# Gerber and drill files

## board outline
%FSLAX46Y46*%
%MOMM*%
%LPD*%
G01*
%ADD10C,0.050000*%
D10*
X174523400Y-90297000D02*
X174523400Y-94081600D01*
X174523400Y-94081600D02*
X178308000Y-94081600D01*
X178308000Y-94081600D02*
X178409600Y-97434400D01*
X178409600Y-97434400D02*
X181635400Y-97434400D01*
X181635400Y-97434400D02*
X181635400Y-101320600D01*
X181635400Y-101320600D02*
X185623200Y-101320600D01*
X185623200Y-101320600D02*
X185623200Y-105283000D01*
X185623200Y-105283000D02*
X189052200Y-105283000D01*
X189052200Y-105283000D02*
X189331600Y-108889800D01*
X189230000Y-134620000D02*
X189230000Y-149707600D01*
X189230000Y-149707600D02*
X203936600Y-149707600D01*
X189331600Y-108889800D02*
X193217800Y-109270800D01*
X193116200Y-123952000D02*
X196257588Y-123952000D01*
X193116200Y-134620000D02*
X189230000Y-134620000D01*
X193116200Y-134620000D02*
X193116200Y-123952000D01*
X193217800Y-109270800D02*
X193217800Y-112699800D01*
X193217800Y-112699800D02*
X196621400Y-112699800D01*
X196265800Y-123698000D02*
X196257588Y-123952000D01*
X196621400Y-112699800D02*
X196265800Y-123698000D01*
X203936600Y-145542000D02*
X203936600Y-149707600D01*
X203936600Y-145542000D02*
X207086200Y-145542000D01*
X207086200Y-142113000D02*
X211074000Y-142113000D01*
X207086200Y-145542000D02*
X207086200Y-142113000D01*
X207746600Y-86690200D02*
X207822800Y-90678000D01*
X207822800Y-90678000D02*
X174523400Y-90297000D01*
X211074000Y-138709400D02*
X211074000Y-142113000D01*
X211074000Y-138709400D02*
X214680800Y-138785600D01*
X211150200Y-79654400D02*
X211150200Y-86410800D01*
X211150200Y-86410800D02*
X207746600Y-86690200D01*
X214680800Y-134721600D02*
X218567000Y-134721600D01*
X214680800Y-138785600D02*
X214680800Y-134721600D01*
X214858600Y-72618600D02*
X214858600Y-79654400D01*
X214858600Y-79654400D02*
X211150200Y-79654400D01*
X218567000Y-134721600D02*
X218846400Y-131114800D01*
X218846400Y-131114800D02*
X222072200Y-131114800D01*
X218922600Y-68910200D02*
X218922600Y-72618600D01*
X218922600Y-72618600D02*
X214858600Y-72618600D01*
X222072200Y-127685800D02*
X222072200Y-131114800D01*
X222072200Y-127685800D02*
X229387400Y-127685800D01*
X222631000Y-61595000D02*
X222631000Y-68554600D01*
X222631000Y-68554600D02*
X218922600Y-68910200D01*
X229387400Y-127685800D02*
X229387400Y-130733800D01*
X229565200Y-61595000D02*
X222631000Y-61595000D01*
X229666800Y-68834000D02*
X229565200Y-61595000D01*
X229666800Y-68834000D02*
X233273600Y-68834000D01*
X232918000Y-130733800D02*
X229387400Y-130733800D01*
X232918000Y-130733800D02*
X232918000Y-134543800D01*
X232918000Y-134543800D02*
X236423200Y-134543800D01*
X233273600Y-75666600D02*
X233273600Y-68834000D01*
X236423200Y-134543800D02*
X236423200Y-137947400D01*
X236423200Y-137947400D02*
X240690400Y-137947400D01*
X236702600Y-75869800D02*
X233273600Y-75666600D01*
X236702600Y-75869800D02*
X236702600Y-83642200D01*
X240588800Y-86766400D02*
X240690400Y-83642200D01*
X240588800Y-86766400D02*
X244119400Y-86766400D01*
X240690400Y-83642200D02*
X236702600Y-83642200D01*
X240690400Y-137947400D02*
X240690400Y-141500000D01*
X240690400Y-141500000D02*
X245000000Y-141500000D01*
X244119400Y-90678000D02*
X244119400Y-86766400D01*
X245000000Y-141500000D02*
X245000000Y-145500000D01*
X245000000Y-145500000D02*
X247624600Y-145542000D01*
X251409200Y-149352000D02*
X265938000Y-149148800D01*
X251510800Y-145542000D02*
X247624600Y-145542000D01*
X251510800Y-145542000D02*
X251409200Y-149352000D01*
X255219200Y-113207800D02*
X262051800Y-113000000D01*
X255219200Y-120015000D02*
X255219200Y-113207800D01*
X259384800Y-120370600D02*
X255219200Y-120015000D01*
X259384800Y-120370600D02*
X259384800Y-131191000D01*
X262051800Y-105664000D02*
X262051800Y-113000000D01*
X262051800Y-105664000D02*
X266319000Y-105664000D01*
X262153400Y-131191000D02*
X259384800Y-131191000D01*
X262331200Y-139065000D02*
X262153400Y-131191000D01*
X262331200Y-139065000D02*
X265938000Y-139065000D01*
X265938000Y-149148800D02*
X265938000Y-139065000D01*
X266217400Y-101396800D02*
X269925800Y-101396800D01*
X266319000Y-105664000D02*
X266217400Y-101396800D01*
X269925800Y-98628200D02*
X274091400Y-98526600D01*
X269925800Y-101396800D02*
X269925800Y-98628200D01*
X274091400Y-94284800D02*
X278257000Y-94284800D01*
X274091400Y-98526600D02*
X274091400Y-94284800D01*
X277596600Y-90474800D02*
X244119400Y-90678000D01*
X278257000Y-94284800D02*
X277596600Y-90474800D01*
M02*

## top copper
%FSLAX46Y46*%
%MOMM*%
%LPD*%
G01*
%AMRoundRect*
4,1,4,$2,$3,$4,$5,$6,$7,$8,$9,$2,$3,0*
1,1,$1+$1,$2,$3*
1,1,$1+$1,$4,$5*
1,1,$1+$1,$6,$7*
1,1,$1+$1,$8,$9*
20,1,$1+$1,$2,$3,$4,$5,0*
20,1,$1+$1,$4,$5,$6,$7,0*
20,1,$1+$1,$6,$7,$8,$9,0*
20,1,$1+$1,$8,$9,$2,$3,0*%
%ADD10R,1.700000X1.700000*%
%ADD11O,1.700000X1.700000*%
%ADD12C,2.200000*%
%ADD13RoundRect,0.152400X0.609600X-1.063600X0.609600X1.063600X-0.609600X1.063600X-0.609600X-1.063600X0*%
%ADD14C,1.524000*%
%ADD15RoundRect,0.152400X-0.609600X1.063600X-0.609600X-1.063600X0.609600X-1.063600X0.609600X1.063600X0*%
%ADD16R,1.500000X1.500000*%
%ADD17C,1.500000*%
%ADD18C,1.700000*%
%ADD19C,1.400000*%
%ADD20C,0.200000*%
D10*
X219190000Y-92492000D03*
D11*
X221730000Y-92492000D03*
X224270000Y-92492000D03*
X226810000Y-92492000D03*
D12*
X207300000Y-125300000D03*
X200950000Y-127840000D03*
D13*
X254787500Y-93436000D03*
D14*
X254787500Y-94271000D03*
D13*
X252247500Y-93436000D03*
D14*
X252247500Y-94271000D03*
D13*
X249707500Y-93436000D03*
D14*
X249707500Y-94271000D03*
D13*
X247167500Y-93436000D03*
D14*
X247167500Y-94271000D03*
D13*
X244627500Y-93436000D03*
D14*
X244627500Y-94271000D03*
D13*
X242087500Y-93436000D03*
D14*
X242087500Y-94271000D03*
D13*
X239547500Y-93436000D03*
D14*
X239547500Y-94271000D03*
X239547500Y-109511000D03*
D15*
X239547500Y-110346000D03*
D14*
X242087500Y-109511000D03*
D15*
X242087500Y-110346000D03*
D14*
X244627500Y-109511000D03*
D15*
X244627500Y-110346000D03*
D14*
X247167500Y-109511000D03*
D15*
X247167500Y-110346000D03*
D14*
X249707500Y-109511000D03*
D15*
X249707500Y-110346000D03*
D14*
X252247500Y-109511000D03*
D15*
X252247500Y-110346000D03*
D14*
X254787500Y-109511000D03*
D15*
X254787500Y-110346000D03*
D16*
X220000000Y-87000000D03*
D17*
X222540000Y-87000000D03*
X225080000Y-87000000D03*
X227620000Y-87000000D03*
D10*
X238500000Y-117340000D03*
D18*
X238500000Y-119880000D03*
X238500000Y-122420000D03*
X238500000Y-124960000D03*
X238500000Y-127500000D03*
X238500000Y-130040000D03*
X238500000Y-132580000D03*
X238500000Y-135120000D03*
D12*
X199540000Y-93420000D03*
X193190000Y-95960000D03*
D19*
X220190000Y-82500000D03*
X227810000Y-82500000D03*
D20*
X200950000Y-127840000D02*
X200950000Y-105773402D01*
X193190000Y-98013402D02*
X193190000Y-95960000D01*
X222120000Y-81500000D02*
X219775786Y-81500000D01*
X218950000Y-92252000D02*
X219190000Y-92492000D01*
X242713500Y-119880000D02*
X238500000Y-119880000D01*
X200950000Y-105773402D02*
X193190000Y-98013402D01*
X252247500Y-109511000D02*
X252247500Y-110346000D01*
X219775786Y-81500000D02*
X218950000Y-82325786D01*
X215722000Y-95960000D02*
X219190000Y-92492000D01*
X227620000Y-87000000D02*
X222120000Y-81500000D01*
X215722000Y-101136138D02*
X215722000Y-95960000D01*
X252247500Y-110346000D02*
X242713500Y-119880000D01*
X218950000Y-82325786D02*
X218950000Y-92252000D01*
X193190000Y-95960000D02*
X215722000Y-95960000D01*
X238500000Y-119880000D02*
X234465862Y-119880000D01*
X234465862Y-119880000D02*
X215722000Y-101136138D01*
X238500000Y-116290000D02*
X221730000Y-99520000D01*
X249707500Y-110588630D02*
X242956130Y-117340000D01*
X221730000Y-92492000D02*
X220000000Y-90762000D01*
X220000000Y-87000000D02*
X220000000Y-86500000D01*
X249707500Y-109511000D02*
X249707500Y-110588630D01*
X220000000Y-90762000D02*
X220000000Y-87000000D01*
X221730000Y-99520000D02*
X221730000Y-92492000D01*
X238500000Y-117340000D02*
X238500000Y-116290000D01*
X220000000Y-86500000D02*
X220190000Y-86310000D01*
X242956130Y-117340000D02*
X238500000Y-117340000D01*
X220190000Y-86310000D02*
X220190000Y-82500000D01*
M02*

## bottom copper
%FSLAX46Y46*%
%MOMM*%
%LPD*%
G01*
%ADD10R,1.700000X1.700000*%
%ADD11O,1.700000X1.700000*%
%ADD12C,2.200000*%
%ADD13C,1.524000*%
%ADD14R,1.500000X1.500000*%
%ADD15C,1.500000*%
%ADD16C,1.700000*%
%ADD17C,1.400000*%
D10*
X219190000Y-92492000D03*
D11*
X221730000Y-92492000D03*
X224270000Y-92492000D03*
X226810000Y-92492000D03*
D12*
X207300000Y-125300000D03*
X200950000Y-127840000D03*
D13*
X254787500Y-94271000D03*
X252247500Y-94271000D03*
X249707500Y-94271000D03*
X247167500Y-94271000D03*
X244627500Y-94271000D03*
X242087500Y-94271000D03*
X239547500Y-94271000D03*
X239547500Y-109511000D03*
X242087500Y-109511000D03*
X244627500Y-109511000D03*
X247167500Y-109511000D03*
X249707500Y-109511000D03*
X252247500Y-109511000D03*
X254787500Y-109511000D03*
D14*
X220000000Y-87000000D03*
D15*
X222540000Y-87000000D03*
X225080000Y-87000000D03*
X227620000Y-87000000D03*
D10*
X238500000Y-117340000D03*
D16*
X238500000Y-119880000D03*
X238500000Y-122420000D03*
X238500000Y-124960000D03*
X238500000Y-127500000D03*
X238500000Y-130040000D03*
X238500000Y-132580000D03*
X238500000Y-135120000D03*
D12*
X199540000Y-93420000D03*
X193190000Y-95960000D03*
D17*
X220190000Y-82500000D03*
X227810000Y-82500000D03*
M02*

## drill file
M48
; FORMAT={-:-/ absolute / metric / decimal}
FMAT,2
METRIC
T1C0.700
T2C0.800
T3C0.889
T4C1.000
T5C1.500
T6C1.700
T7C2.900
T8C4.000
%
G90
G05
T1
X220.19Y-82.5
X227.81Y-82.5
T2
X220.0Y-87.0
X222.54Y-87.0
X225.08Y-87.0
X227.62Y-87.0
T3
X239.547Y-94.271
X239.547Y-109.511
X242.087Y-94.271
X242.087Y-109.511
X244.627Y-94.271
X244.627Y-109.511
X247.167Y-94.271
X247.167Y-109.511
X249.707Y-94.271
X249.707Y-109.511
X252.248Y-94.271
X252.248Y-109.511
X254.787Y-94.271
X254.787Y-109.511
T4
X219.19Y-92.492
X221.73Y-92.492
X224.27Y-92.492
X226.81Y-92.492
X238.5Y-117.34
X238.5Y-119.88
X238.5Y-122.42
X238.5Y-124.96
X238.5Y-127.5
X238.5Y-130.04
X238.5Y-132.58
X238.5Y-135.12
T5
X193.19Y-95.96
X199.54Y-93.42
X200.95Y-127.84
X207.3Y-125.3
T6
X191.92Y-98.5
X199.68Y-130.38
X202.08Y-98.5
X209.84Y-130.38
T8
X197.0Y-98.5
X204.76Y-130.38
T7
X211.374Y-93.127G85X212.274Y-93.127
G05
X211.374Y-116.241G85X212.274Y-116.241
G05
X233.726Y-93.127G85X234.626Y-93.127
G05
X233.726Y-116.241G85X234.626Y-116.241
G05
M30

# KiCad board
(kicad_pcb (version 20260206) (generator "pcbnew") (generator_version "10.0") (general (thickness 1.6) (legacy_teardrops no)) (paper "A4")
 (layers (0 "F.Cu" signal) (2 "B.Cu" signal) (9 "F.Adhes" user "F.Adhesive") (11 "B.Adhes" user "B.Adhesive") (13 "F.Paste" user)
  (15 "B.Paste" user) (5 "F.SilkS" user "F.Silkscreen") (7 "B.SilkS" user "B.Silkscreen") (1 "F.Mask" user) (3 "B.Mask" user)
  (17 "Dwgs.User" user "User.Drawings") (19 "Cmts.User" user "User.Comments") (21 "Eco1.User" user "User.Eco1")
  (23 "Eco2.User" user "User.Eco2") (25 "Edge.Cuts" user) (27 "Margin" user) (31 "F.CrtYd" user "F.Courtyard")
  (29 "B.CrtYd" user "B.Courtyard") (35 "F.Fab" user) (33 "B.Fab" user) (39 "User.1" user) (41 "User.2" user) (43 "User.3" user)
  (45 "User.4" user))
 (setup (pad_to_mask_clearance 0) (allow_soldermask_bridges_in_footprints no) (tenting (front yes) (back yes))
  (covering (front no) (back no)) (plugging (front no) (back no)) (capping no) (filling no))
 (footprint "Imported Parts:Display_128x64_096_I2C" (layer "F.Cu") (at 223 92.492)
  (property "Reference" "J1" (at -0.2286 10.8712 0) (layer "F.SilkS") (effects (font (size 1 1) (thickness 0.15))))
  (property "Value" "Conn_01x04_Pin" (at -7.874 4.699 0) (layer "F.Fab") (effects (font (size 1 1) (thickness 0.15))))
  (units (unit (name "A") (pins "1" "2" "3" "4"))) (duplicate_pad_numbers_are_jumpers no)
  (pad "" np_thru_hole oval (at -11.176 0.635) (size 3.8 2.9) (drill oval 3.8 2.9) (layers "*.Cu" "*.Mask"))
  (pad "" np_thru_hole oval (at -11.176 23.749) (size 3.8 2.9) (drill oval 3.8 2.9) (layers "*.Cu" "*.Mask"))
  (pad "" np_thru_hole oval (at 11.176 0.635) (size 3.8 2.9) (drill oval 3.8 2.9) (layers "*.Cu" "*.Mask"))
  (pad "" np_thru_hole oval (at 11.176 23.749) (size 3.8 2.9) (drill oval 3.8 2.9) (layers "*.Cu" "*.Mask"))
  (pad "1" thru_hole rect (at -3.81 0 90) (size 1.7 1.7) (drill 1) (layers "*.Cu" "*.Mask") (remove_unused_layers no) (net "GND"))
  (pad "2" thru_hole oval (at -1.27 0 90) (size 1.7 1.7) (drill 1) (layers "*.Cu" "*.Mask") (remove_unused_layers no) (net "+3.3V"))
  (pad "3" thru_hole oval (at 1.27 0 90) (size 1.7 1.7) (drill 1) (layers "*.Cu" "*.Mask") (remove_unused_layers no)
   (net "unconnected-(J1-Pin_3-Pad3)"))
  (pad "4" thru_hole oval (at 3.81 0 90) (size 1.7 1.7) (drill 1) (layers "*.Cu" "*.Mask") (remove_unused_layers no)
   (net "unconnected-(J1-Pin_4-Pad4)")))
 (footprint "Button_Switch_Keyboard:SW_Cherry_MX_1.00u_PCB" (layer "F.Cu") (at 207.3 125.3)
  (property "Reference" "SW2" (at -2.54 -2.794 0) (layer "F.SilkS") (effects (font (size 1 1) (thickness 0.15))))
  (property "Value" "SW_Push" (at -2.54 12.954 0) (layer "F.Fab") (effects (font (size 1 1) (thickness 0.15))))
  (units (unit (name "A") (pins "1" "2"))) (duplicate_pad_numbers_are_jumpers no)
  (pad "" np_thru_hole circle (at -7.62 5.08) (size 1.7 1.7) (drill 1.7) (layers "*.Cu" "*.Mask"))
  (pad "" np_thru_hole circle (at -2.54 5.08) (size 4 4) (drill 4) (layers "*.Cu" "*.Mask"))
  (pad "" np_thru_hole circle (at 2.54 5.08) (size 1.7 1.7) (drill 1.7) (layers "*.Cu" "*.Mask"))
  (pad "1" thru_hole circle (at 0 0) (size 2.2 2.2) (drill 1.5) (layers "*.Cu" "*.Mask") (remove_unused_layers no)
   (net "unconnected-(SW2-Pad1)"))
  (pad "2" thru_hole circle (at -6.35 2.54) (size 2.2 2.2) (drill 1.5) (layers "*.Cu" "*.Mask") (remove_unused_layers no) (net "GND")))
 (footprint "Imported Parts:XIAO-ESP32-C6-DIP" (layer "F.Cu") (at 247.1675 101.891)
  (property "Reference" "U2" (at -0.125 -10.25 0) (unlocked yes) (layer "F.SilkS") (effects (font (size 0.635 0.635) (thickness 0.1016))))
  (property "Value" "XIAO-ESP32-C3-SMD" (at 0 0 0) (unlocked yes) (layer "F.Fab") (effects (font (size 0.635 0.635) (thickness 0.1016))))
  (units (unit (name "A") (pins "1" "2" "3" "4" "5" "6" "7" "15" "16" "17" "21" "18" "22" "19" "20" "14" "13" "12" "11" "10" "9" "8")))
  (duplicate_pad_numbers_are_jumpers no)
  (pad "1" smd roundrect (at 7.62 -8.455 90) (size 2.432 1.524) (layers "F.Cu" "F.Mask") (roundrect_rratio 0.1)
   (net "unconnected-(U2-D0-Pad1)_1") (thermal_bridge_angle 45))
  (pad "1" thru_hole circle (at 7.62 -7.62 90) (size 1.524 1.524) (drill 0.889) (layers "*.Cu" "*.Mask") (remove_unused_layers no)
   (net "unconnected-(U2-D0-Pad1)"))
  (pad "2" smd roundrect (at 5.08 -8.455 90) (size 2.432 1.524) (layers "F.Cu" "F.Mask") (roundrect_rratio 0.1)
   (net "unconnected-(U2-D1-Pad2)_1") (thermal_bridge_angle 45))
  (pad "2" thru_hole circle (at 5.08 -7.62 90) (size 1.524 1.524) (drill 0.889) (layers "*.Cu" "*.Mask") (remove_unused_layers no)
   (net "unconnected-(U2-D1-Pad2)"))
  (pad "3" smd roundrect (at 2.54 -8.455 90) (size 2.432 1.524) (layers "F.Cu" "F.Mask") (roundrect_rratio 0.1)
   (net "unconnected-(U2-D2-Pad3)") (thermal_bridge_angle 45))
  (pad "3" thru_hole circle (at 2.54 -7.62 90) (size 1.524 1.524) (drill 0.889) (layers "*.Cu" "*.Mask") (remove_unused_layers no)
   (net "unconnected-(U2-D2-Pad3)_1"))
  (pad "4" smd roundrect (at 0 -8.455 90) (size 2.432 1.524) (layers "F.Cu" "F.Mask") (roundrect_rratio 0.1)
   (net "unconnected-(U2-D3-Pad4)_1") (thermal_bridge_angle 45))
  (pad "4" thru_hole circle (at 0 -7.62 90) (size 1.524 1.524) (drill 0.889) (layers "*.Cu" "*.Mask") (remove_unused_layers no)
   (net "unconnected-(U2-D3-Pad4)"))
  (pad "5" smd roundrect (at -2.54 -8.455 90) (size 2.432 1.524) (layers "F.Cu" "F.Mask") (roundrect_rratio 0.1)
   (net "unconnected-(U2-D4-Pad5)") (thermal_bridge_angle 45))
  (pad "5" thru_hole circle (at -2.54 -7.62 90) (size 1.524 1.524) (drill 0.889) (layers "*.Cu" "*.Mask") (remove_unused_layers no)
   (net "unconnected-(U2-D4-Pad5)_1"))
  (pad "6" smd roundrect (at -5.08 -8.455 90) (size 2.432 1.524) (layers "F.Cu" "F.Mask") (roundrect_rratio 0.1)
   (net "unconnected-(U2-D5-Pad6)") (thermal_bridge_angle 45))
  (pad "6" thru_hole circle (at -5.08 -7.62 90) (size 1.524 1.524) (drill 0.889) (layers "*.Cu" "*.Mask") (remove_unused_layers no)
   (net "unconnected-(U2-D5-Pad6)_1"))
  (pad "7" smd roundrect (at -7.62 -8.455 90) (size 2.432 1.524) (layers "F.Cu" "F.Mask") (roundrect_rratio 0.1)
   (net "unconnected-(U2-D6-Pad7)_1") (thermal_bridge_angle 45))
  (pad "7" thru_hole circle (at -7.62 -7.62 90) (size 1.524 1.524) (drill 0.889) (layers "*.Cu" "*.Mask") (remove_unused_layers no)
   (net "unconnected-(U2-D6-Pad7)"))
  (pad "8" thru_hole circle (at -7.62 7.62 270) (size 1.524 1.524) (drill 0.889) (layers "*.Cu" "*.Mask") (remove_unused_layers no)
   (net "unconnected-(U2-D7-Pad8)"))
  (pad "8" smd roundrect (at -7.62 8.455 270) (size 2.432 1.524) (layers "F.Cu" "F.Mask") (roundrect_rratio 0.1)
   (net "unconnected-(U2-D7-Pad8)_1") (thermal_bridge_angle 45))
  (pad "9" thru_hole circle (at -5.08 7.62 270) (size 1.524 1.524) (drill 0.889) (layers "*.Cu" "*.Mask") (remove_unused_layers no)
   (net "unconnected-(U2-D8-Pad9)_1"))
  (pad "9" smd roundrect (at -5.08 8.455 270) (size 2.432 1.524) (layers "F.Cu" "F.Mask") (roundrect_rratio 0.1)
   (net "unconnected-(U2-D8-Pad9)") (thermal_bridge_angle 45))
  (pad "10" thru_hole circle (at -2.54 7.62 270) (size 1.524 1.524) (drill 0.889) (layers "*.Cu" "*.Mask") (remove_unused_layers no)
   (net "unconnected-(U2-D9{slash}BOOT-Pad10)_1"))
  (pad "10" smd roundrect (at -2.54 8.455 270) (size 2.432 1.524) (layers "F.Cu" "F.Mask") (roundrect_rratio 0.1)
   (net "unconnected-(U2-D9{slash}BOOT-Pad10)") (thermal_bridge_angle 45))
  (pad "11" thru_hole circle (at 0 7.62 270) (size 1.524 1.524) (drill 0.889) (layers "*.Cu" "*.Mask") (remove_unused_layers no)
   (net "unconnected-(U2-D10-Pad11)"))
  (pad "11" smd roundrect (at 0 8.455 270) (size 2.432 1.524) (layers "F.Cu" "F.Mask") (roundrect_rratio 0.1)
   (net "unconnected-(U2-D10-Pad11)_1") (thermal_bridge_angle 45))
  (pad "12" thru_hole circle (at 2.54 7.62 270) (size 1.524 1.524) (drill 0.889) (layers "*.Cu" "*.Mask") (remove_unused_layers no)
   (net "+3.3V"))
  (pad "12" smd roundrect (at 2.54 8.455 270) (size 2.432 1.524) (layers "F.Cu" "F.Mask") (roundrect_rratio 0.1) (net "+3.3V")
   (thermal_bridge_angle 45))
  (pad "13" thru_hole circle (at 5.08 7.62 270) (size 1.524 1.524) (drill 0.889) (layers "*.Cu" "*.Mask") (remove_unused_layers no)
   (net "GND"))
  (pad "13" smd roundrect (at 5.08 8.455 270) (size 2.432 1.524) (layers "F.Cu" "F.Mask") (roundrect_rratio 0.1) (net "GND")
   (thermal_bridge_angle 45))
  (pad "14" thru_hole circle (at 7.62 7.62 270) (size 1.524 1.524) (drill 0.889) (layers "*.Cu" "*.Mask") (remove_unused_layers no)
   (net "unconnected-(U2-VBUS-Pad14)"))
  (pad "14" smd roundrect (at 7.62 8.455 270) (size 2.432 1.524) (layers "F.Cu" "F.Mask") (roundrect_rratio 0.1)
   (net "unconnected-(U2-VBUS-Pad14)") (thermal_bridge_angle 45)))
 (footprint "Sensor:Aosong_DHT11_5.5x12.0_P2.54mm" (layer "F.Cu") (at 220 87 90)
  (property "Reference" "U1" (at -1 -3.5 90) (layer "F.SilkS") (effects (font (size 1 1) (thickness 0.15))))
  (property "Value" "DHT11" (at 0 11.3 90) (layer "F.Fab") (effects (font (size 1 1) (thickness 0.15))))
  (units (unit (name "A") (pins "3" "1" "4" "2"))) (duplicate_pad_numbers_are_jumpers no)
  (pad "1" thru_hole rect (at 0 0 90) (size 1.5 1.5) (drill 0.8) (layers "*.Cu" "*.Mask") (remove_unused_layers no) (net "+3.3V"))
  (pad "2" thru_hole circle (at 0 2.54 90) (size 1.5 1.5) (drill 0.8) (layers "*.Cu" "*.Mask") (remove_unused_layers no)
   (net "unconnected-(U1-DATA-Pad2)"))
  (pad "3" thru_hole circle (at 0 5.08 90) (size 1.5 1.5) (drill 0.8) (layers "*.Cu" "*.Mask") (remove_unused_layers no)
   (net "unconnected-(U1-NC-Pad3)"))
  (pad "4" thru_hole circle (at 0 7.62 90) (size 1.5 1.5) (drill 0.8) (layers "*.Cu" "*.Mask") (remove_unused_layers no) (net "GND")))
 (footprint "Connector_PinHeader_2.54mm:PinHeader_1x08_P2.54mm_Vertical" (layer "F.Cu") (at 238.5 117.34)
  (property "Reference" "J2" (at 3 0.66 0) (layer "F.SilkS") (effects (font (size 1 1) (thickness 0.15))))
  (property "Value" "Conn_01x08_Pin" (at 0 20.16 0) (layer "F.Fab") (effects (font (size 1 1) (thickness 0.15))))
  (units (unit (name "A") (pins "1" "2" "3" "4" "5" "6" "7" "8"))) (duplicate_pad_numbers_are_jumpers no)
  (pad "1" thru_hole rect (at 0 0) (size 1.7 1.7) (drill 1) (layers "*.Cu" "*.Mask") (remove_unused_layers no) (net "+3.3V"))
  (pad "2" thru_hole circle (at 0 2.54) (size 1.7 1.7) (drill 1) (layers "*.Cu" "*.Mask") (remove_unused_layers no) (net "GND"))
  (pad "3" thru_hole circle (at 0 5.08) (size 1.7 1.7) (drill 1) (layers "*.Cu" "*.Mask") (remove_unused_layers no)
   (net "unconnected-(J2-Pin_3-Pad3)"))
  (pad "4" thru_hole circle (at 0 7.62) (size 1.7 1.7) (drill 1) (layers "*.Cu" "*.Mask") (remove_unused_layers no)
   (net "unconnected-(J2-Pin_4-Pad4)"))
  (pad "5" thru_hole circle (at 0 10.16) (size 1.7 1.7) (drill 1) (layers "*.Cu" "*.Mask") (remove_unused_layers no)
   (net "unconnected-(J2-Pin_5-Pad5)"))
  (pad "6" thru_hole circle (at 0 12.7) (size 1.7 1.7) (drill 1) (layers "*.Cu" "*.Mask") (remove_unused_layers no)
   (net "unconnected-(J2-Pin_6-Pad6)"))
  (pad "7" thru_hole circle (at 0 15.24) (size 1.7 1.7) (drill 1) (layers "*.Cu" "*.Mask") (remove_unused_layers no)
   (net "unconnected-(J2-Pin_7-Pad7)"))
  (pad "8" thru_hole circle (at 0 17.78) (size 1.7 1.7) (drill 1) (layers "*.Cu" "*.Mask") (remove_unused_layers no)
   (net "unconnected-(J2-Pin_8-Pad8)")))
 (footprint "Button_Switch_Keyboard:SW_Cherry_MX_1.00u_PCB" (layer "F.Cu") (at 199.54 93.42)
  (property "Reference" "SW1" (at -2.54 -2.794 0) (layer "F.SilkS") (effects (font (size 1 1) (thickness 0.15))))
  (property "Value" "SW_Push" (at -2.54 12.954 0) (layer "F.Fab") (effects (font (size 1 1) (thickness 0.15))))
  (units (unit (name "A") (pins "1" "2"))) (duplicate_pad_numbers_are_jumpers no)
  (pad "" np_thru_hole circle (at -7.62 5.08) (size 1.7 1.7) (drill 1.7) (layers "*.Cu" "*.Mask"))
  (pad "" np_thru_hole circle (at -2.54 5.08) (size 4 4) (drill 4) (layers "*.Cu" "*.Mask"))
  (pad "" np_thru_hole circle (at 2.54 5.08) (size 1.7 1.7) (drill 1.7) (layers "*.Cu" "*.Mask"))
  (pad "1" thru_hole circle (at 0 0) (size 2.2 2.2) (drill 1.5) (layers "*.Cu" "*.Mask") (remove_unused_layers no)
   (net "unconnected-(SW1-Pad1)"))
  (pad "2" thru_hole circle (at -6.35 2.54) (size 2.2 2.2) (drill 1.5) (layers "*.Cu" "*.Mask") (remove_unused_layers no) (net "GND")))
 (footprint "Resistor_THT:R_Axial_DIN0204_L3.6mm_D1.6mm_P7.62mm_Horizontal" (layer "F.Cu") (at 220.19 82.5)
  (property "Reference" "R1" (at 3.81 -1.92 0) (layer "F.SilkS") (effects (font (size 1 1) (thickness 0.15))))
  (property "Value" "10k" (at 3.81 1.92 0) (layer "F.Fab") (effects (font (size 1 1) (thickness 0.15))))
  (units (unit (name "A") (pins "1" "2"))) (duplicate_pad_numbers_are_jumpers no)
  (pad "1" thru_hole circle (at 0 0) (size 1.4 1.4) (drill 0.7) (layers "*.Cu" "*.Mask") (remove_unused_layers no) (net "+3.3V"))
  (pad "2" thru_hole circle (at 7.62 0) (size 1.4 1.4) (drill 0.7) (layers "*.Cu" "*.Mask") (remove_unused_layers no)
   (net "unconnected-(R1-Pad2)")))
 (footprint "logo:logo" (layer "F.Cu") (at 225.5 74.5)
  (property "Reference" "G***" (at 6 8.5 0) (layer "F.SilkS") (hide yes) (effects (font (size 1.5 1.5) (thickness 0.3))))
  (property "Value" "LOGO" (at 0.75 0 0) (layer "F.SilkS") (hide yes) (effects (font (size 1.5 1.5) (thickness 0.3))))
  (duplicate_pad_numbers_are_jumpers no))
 (gr_line (start 174.5234 90.297) (end 174.5234 94.0816) (stroke (width 0.05) (type default)) (locked yes) (layer "Edge.Cuts"))
 (gr_line (start 174.5234 94.0816) (end 178.308 94.0816) (stroke (width 0.05) (type default)) (locked yes) (layer "Edge.Cuts"))
 (gr_line (start 178.308 94.0816) (end 178.4096 97.4344) (stroke (width 0.05) (type default)) (locked yes) (layer "Edge.Cuts"))
 (gr_line (start 178.4096 97.4344) (end 181.6354 97.4344) (stroke (width 0.05) (type default)) (locked yes) (layer "Edge.Cuts"))
 (gr_line (start 181.6354 97.4344) (end 181.6354 101.3206) (stroke (width 0.05) (type default)) (locked yes) (layer "Edge.Cuts"))
 (gr_line (start 181.6354 101.3206) (end 185.6232 101.3206) (stroke (width 0.05) (type default)) (locked yes) (layer "Edge.Cuts"))
 (gr_line (start 185.6232 101.3206) (end 185.6232 105.283) (stroke (width 0.05) (type default)) (locked yes) (layer "Edge.Cuts"))
 (gr_line (start 185.6232 105.283) (end 189.0522 105.283) (stroke (width 0.05) (type default)) (locked yes) (layer "Edge.Cuts"))
 (gr_line (start 189.0522 105.283) (end 189.3316 108.8898) (stroke (width 0.05) (type default)) (locked yes) (layer "Edge.Cuts"))
 (gr_line (start 189.23 134.62) (end 189.23 149.7076) (stroke (width 0.05) (type default)) (locked yes) (layer "Edge.Cuts"))
 (gr_line (start 189.23 149.7076) (end 203.9366 149.7076) (stroke (width 0.05) (type default)) (locked yes) (layer "Edge.Cuts"))
 (gr_line (start 189.3316 108.8898) (end 193.2178 109.2708) (stroke (width 0.05) (type default)) (locked yes) (layer "Edge.Cuts"))
 (gr_line (start 193.1162 123.952) (end 196.257588 123.952) (stroke (width 0.05) (type default)) (locked yes) (layer "Edge.Cuts"))
 (gr_line (start 193.1162 134.62) (end 189.23 134.62) (stroke (width 0.05) (type default)) (locked yes) (layer "Edge.Cuts"))
 (gr_line (start 193.1162 134.62) (end 193.1162 123.952) (stroke (width 0.05) (type default)) (locked yes) (layer "Edge.Cuts"))
 (gr_line (start 193.2178 109.2708) (end 193.2178 112.6998) (stroke (width 0.05) (type default)) (locked yes) (layer "Edge.Cuts"))
 (gr_line (start 193.2178 112.6998) (end 196.6214 112.6998) (stroke (width 0.05) (type default)) (locked yes) (layer "Edge.Cuts"))
 (gr_line (start 196.2658 123.698) (end 196.257588 123.952) (stroke (width 0.05) (type default)) (layer "Edge.Cuts"))
 (gr_line (start 196.6214 112.6998) (end 196.2658 123.698) (stroke (width 0.05) (type default)) (locked yes) (layer "Edge.Cuts"))
 (gr_line (start 203.9366 145.542) (end 203.9366 149.7076) (stroke (width 0.05) (type default)) (locked yes) (layer "Edge.Cuts"))
 (gr_line (start 203.9366 145.542) (end 207.0862 145.542) (stroke (width 0.05) (type default)) (locked yes) (layer "Edge.Cuts"))
 (gr_line (start 207.0862 142.113) (end 211.074 142.113) (stroke (width 0.05) (type default)) (locked yes) (layer "Edge.Cuts"))
 (gr_line (start 207.0862 145.542) (end 207.0862 142.113) (stroke (width 0.05) (type default)) (locked yes) (layer "Edge.Cuts"))
 (gr_line (start 207.7466 86.6902) (end 207.8228 90.678) (stroke (width 0.05) (type default)) (locked yes) (layer "Edge.Cuts"))
 (gr_line (start 207.8228 90.678) (end 174.5234 90.297) (stroke (width 0.05) (type default)) (locked yes) (layer "Edge.Cuts"))
 (gr_line (start 211.074 138.7094) (end 211.074 142.113) (stroke (width 0.05) (type default)) (locked yes) (layer "Edge.Cuts"))
 (gr_line (start 211.074 138.7094) (end 214.6808 138.7856) (stroke (width 0.05) (type default)) (locked yes) (layer "Edge.Cuts"))
 (gr_line (start 211.1502 79.6544) (end 211.1502 86.4108) (stroke (width 0.05) (type default)) (locked yes) (layer "Edge.Cuts"))
 (gr_line (start 211.1502 86.4108) (end 207.7466 86.6902) (stroke (width 0.05) (type default)) (locked yes) (layer "Edge.Cuts"))
 (gr_line (start 214.6808 134.7216) (end 218.567 134.7216) (stroke (width 0.05) (type default)) (locked yes) (layer "Edge.Cuts"))
 (gr_line (start 214.6808 138.7856) (end 214.6808 134.7216) (stroke (width 0.05) (type default)) (locked yes) (layer "Edge.Cuts"))
 (gr_line (start 214.8586 72.6186) (end 214.8586 79.6544) (stroke (width 0.05) (type default)) (locked yes) (layer "Edge.Cuts"))
 (gr_line (start 214.8586 79.6544) (end 211.1502 79.6544) (stroke (width 0.05) (type default)) (locked yes) (layer "Edge.Cuts"))
 (gr_line (start 218.567 134.7216) (end 218.8464 131.1148) (stroke (width 0.05) (type default)) (locked yes) (layer "Edge.Cuts"))
 (gr_line (start 218.8464 131.1148) (end 222.0722 131.1148) (stroke (width 0.05) (type default)) (locked yes) (layer "Edge.Cuts"))
 (gr_line (start 218.9226 68.9102) (end 218.9226 72.6186) (stroke (width 0.05) (type default)) (locked yes) (layer "Edge.Cuts"))
 (gr_line (start 218.9226 72.6186) (end 214.8586 72.6186) (stroke (width 0.05) (type default)) (locked yes) (layer "Edge.Cuts"))
 (gr_line (start 222.0722 127.6858) (end 222.0722 131.1148) (stroke (width 0.05) (type default)) (locked yes) (layer "Edge.Cuts"))
 (gr_line (start 222.0722 127.6858) (end 229.3874 127.6858) (stroke (width 0.05) (type default)) (locked yes) (layer "Edge.Cuts"))
 (gr_line (start 222.631 61.595) (end 222.631 68.5546) (stroke (width 0.05) (type default)) (locked yes) (layer "Edge.Cuts"))
 (gr_line (start 222.631 68.5546) (end 218.9226 68.9102) (stroke (width 0.05) (type default)) (locked yes) (layer "Edge.Cuts"))
 (gr_line (start 229.3874 127.6858) (end 229.3874 130.7338) (stroke (width 0.05) (type default)) (locked yes) (layer "Edge.Cuts"))
 (gr_line (start 229.5652 61.595) (end 222.631 61.595) (stroke (width 0.05) (type default)) (locked yes) (layer "Edge.Cuts"))
 (gr_line (start 229.6668 68.834) (end 229.5652 61.595) (stroke (width 0.05) (type default)) (locked yes) (layer "Edge.Cuts"))
 (gr_line (start 229.6668 68.834) (end 233.2736 68.834) (stroke (width 0.05) (type default)) (locked yes) (layer "Edge.Cuts"))
 (gr_line (start 232.918 130.7338) (end 229.3874 130.7338) (stroke (width 0.05) (type default)) (locked yes) (layer "Edge.Cuts"))
 (gr_line (start 232.918 130.7338) (end 232.918 134.5438) (stroke (width 0.05) (type default)) (locked yes) (layer "Edge.Cuts"))
 (gr_line (start 232.918 134.5438) (end 236.4232 134.5438) (stroke (width 0.05) (type default)) (locked yes) (layer "Edge.Cuts"))
 (gr_line (start 233.2736 75.6666) (end 233.2736 68.834) (stroke (width 0.05) (type default)) (locked yes) (layer "Edge.Cuts"))
 (gr_line (start 236.4232 134.5438) (end 236.4232 137.9474) (stroke (width 0.05) (type default)) (locked yes) (layer "Edge.Cuts"))
 (gr_line (start 236.4232 137.9474) (end 240.6904 137.9474) (stroke (width 0.05) (type default)) (locked yes) (layer "Edge.Cuts"))
 (gr_line (start 236.7026 75.8698) (end 233.2736 75.6666) (stroke (width 0.05) (type default)) (locked yes) (layer "Edge.Cuts"))
 (gr_line (start 236.7026 75.8698) (end 236.7026 83.6422) (stroke (width 0.05) (type default)) (locked yes) (layer "Edge.Cuts"))
 (gr_line (start 240.5888 86.7664) (end 240.6904 83.6422) (stroke (width 0.05) (type default)) (locked yes) (layer "Edge.Cuts"))
 (gr_line (start 240.5888 86.7664) (end 244.1194 86.7664) (stroke (width 0.05) (type default)) (locked yes) (layer "Edge.Cuts"))
 (gr_line (start 240.6904 83.6422) (end 236.7026 83.6422) (stroke (width 0.05) (type default)) (locked yes) (layer "Edge.Cuts"))
 (gr_line (start 240.6904 137.9474) (end 240.6904 141.5) (stroke (width 0.05) (type default)) (layer "Edge.Cuts"))
 (gr_line (start 240.6904 141.5) (end 245 141.5) (stroke (width 0.05) (type default)) (layer "Edge.Cuts"))
 (gr_line (start 244.1194 90.678) (end 244.1194 86.7664) (stroke (width 0.05) (type default)) (locked yes) (layer "Edge.Cuts"))
 (gr_line (start 245 141.5) (end 245 145.5) (stroke (width 0.05) (type default)) (layer "Edge.Cuts"))
 (gr_line (start 245 145.5) (end 247.6246 145.542) (stroke (width 0.05) (type default)) (layer "Edge.Cuts"))
 (gr_line (start 251.4092 149.352) (end 265.938 149.1488) (stroke (width 0.05) (type default)) (locked yes) (layer "Edge.Cuts"))
 (gr_line (start 251.5108 145.542) (end 247.6246 145.542) (stroke (width 0.05) (type default)) (locked yes) (layer "Edge.Cuts"))
 (gr_line (start 251.5108 145.542) (end 251.4092 149.352) (stroke (width 0.05) (type default)) (locked yes) (layer "Edge.Cuts"))
 (gr_line (start 255.2192 113.2078) (end 262.0518 113) (stroke (width 0.05) (type default)) (layer "Edge.Cuts"))
 (gr_line (start 255.2192 120.015) (end 255.2192 113.2078) (stroke (width 0.05) (type default)) (locked yes) (layer "Edge.Cuts"))
 (gr_line (start 259.3848 120.3706) (end 255.2192 120.015) (stroke (width 0.05) (type default)) (locked yes) (layer "Edge.Cuts"))
 (gr_line (start 259.3848 120.3706) (end 259.3848 131.191) (stroke (width 0.05) (type default)) (locked yes) (layer "Edge.Cuts"))
 (gr_line (start 262.0518 105.664) (end 262.0518 113) (stroke (width 0.05) (type default)) (layer "Edge.Cuts"))
 (gr_line (start 262.0518 105.664) (end 266.319 105.664) (stroke (width 0.05) (type default)) (locked yes) (layer "Edge.Cuts"))
 (gr_line (start 262.1534 131.191) (end 259.3848 131.191) (stroke (width 0.05) (type default)) (locked yes) (layer "Edge.Cuts"))
 (gr_line (start 262.3312 139.065) (end 262.1534 131.191) (stroke (width 0.05) (type default)) (locked yes) (layer "Edge.Cuts"))
 (gr_line (start 262.3312 139.065) (end 265.938 139.065) (stroke (width 0.05) (type default)) (locked yes) (layer "Edge.Cuts"))
 (gr_line (start 265.938 149.1488) (end 265.938 139.065) (stroke (width 0.05) (type default)) (locked yes) (layer "Edge.Cuts"))
 (gr_line (start 266.2174 101.3968) (end 269.9258 101.3968) (stroke (width 0.05) (type default)) (locked yes) (layer "Edge.Cuts"))
 (gr_line (start 266.319 105.664) (end 266.2174 101.3968) (stroke (width 0.05) (type default)) (locked yes) (layer "Edge.Cuts"))
 (gr_line (start 269.9258 98.6282) (end 274.0914 98.5266) (stroke (width 0.05) (type default)) (locked yes) (layer "Edge.Cuts"))
 (gr_line (start 269.9258 101.3968) (end 269.9258 98.6282) (stroke (width 0.05) (type default)) (locked yes) (layer "Edge.Cuts"))
 (gr_line (start 274.0914 94.2848) (end 278.257 94.2848) (stroke (width 0.05) (type default)) (locked yes) (layer "Edge.Cuts"))
 (gr_line (start 274.0914 98.5266) (end 274.0914 94.2848) (stroke (width 0.05) (type default)) (locked yes) (layer "Edge.Cuts"))
 (gr_line (start 277.5966 90.4748) (end 244.1194 90.678) (stroke (width 0.05) (type default)) (locked yes) (layer "Edge.Cuts"))
 (gr_line (start 278.257 94.2848) (end 277.5966 90.4748) (stroke (width 0.05) (type default)) (locked yes) (layer "Edge.Cuts"))
 (segment (start 200.95 127.84) (end 200.95 105.773402) (width 0.2) (layer "F.Cu") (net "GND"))
 (segment (start 193.19 98.013402) (end 193.19 95.96) (width 0.2) (layer "F.Cu") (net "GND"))
 (segment (start 222.12 81.5) (end 219.775786 81.5) (width 0.2) (layer "F.Cu") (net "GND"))
 (segment (start 218.95 92.252) (end 219.19 92.492) (width 0.2) (layer "F.Cu") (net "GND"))
 (segment (start 242.7135 119.88) (end 238.5 119.88) (width 0.2) (layer "F.Cu") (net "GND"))
 (segment (start 200.95 105.773402) (end 193.19 98.013402) (width 0.2) (layer "F.Cu") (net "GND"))
 (segment (start 252.2475 109.511) (end 252.2475 110.346) (width 0.2) (layer "F.Cu") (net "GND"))
 (segment (start 219.775786 81.5) (end 218.95 82.325786) (width 0.2) (layer "F.Cu") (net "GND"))
 (segment (start 215.722 95.96) (end 219.19 92.492) (width 0.2) (layer "F.Cu") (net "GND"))
 (segment (start 227.62 87) (end 222.12 81.5) (width 0.2) (layer "F.Cu") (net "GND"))
 (segment (start 215.722 101.136138) (end 215.722 95.96) (width 0.2) (layer "F.Cu") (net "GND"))
 (segment (start 252.2475 110.346) (end 242.7135 119.88) (width 0.2) (layer "F.Cu") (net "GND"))
 (segment (start 218.95 82.325786) (end 218.95 92.252) (width 0.2) (layer "F.Cu") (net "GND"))
 (segment (start 193.19 95.96) (end 215.722 95.96) (width 0.2) (layer "F.Cu") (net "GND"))
 (segment (start 238.5 119.88) (end 234.465862 119.88) (width 0.2) (layer "F.Cu") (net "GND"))
 (segment (start 234.465862 119.88) (end 215.722 101.136138) (width 0.2) (layer "F.Cu") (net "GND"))
 (segment (start 238.5 116.29) (end 221.73 99.52) (width 0.2) (layer "F.Cu") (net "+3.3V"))
 (segment (start 249.7075 110.58863) (end 242.95613 117.34) (width 0.2) (layer "F.Cu") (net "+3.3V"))
 (segment (start 221.73 92.492) (end 220 90.762) (width 0.2) (layer "F.Cu") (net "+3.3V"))
 (segment (start 220 87) (end 220 86.5) (width 0.2) (layer "F.Cu") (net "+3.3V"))
 (segment (start 249.7075 109.511) (end 249.7075 110.58863) (width 0.2) (layer "F.Cu") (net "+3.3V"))
 (segment (start 220 90.762) (end 220 87) (width 0.2) (layer "F.Cu") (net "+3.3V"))
 (segment (start 221.73 99.52) (end 221.73 92.492) (width 0.2) (layer "F.Cu") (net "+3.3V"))
 (segment (start 238.5 117.34) (end 238.5 116.29) (width 0.2) (layer "F.Cu") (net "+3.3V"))
 (segment (start 220 86.5) (end 220.19 86.31) (width 0.2) (layer "F.Cu") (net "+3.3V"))
 (segment (start 242.95613 117.34) (end 238.5 117.34) (width 0.2) (layer "F.Cu") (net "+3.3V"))
 (segment (start 220.19 86.31) (end 220.19 82.5) (width 0.2) (layer "F.Cu") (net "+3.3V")))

